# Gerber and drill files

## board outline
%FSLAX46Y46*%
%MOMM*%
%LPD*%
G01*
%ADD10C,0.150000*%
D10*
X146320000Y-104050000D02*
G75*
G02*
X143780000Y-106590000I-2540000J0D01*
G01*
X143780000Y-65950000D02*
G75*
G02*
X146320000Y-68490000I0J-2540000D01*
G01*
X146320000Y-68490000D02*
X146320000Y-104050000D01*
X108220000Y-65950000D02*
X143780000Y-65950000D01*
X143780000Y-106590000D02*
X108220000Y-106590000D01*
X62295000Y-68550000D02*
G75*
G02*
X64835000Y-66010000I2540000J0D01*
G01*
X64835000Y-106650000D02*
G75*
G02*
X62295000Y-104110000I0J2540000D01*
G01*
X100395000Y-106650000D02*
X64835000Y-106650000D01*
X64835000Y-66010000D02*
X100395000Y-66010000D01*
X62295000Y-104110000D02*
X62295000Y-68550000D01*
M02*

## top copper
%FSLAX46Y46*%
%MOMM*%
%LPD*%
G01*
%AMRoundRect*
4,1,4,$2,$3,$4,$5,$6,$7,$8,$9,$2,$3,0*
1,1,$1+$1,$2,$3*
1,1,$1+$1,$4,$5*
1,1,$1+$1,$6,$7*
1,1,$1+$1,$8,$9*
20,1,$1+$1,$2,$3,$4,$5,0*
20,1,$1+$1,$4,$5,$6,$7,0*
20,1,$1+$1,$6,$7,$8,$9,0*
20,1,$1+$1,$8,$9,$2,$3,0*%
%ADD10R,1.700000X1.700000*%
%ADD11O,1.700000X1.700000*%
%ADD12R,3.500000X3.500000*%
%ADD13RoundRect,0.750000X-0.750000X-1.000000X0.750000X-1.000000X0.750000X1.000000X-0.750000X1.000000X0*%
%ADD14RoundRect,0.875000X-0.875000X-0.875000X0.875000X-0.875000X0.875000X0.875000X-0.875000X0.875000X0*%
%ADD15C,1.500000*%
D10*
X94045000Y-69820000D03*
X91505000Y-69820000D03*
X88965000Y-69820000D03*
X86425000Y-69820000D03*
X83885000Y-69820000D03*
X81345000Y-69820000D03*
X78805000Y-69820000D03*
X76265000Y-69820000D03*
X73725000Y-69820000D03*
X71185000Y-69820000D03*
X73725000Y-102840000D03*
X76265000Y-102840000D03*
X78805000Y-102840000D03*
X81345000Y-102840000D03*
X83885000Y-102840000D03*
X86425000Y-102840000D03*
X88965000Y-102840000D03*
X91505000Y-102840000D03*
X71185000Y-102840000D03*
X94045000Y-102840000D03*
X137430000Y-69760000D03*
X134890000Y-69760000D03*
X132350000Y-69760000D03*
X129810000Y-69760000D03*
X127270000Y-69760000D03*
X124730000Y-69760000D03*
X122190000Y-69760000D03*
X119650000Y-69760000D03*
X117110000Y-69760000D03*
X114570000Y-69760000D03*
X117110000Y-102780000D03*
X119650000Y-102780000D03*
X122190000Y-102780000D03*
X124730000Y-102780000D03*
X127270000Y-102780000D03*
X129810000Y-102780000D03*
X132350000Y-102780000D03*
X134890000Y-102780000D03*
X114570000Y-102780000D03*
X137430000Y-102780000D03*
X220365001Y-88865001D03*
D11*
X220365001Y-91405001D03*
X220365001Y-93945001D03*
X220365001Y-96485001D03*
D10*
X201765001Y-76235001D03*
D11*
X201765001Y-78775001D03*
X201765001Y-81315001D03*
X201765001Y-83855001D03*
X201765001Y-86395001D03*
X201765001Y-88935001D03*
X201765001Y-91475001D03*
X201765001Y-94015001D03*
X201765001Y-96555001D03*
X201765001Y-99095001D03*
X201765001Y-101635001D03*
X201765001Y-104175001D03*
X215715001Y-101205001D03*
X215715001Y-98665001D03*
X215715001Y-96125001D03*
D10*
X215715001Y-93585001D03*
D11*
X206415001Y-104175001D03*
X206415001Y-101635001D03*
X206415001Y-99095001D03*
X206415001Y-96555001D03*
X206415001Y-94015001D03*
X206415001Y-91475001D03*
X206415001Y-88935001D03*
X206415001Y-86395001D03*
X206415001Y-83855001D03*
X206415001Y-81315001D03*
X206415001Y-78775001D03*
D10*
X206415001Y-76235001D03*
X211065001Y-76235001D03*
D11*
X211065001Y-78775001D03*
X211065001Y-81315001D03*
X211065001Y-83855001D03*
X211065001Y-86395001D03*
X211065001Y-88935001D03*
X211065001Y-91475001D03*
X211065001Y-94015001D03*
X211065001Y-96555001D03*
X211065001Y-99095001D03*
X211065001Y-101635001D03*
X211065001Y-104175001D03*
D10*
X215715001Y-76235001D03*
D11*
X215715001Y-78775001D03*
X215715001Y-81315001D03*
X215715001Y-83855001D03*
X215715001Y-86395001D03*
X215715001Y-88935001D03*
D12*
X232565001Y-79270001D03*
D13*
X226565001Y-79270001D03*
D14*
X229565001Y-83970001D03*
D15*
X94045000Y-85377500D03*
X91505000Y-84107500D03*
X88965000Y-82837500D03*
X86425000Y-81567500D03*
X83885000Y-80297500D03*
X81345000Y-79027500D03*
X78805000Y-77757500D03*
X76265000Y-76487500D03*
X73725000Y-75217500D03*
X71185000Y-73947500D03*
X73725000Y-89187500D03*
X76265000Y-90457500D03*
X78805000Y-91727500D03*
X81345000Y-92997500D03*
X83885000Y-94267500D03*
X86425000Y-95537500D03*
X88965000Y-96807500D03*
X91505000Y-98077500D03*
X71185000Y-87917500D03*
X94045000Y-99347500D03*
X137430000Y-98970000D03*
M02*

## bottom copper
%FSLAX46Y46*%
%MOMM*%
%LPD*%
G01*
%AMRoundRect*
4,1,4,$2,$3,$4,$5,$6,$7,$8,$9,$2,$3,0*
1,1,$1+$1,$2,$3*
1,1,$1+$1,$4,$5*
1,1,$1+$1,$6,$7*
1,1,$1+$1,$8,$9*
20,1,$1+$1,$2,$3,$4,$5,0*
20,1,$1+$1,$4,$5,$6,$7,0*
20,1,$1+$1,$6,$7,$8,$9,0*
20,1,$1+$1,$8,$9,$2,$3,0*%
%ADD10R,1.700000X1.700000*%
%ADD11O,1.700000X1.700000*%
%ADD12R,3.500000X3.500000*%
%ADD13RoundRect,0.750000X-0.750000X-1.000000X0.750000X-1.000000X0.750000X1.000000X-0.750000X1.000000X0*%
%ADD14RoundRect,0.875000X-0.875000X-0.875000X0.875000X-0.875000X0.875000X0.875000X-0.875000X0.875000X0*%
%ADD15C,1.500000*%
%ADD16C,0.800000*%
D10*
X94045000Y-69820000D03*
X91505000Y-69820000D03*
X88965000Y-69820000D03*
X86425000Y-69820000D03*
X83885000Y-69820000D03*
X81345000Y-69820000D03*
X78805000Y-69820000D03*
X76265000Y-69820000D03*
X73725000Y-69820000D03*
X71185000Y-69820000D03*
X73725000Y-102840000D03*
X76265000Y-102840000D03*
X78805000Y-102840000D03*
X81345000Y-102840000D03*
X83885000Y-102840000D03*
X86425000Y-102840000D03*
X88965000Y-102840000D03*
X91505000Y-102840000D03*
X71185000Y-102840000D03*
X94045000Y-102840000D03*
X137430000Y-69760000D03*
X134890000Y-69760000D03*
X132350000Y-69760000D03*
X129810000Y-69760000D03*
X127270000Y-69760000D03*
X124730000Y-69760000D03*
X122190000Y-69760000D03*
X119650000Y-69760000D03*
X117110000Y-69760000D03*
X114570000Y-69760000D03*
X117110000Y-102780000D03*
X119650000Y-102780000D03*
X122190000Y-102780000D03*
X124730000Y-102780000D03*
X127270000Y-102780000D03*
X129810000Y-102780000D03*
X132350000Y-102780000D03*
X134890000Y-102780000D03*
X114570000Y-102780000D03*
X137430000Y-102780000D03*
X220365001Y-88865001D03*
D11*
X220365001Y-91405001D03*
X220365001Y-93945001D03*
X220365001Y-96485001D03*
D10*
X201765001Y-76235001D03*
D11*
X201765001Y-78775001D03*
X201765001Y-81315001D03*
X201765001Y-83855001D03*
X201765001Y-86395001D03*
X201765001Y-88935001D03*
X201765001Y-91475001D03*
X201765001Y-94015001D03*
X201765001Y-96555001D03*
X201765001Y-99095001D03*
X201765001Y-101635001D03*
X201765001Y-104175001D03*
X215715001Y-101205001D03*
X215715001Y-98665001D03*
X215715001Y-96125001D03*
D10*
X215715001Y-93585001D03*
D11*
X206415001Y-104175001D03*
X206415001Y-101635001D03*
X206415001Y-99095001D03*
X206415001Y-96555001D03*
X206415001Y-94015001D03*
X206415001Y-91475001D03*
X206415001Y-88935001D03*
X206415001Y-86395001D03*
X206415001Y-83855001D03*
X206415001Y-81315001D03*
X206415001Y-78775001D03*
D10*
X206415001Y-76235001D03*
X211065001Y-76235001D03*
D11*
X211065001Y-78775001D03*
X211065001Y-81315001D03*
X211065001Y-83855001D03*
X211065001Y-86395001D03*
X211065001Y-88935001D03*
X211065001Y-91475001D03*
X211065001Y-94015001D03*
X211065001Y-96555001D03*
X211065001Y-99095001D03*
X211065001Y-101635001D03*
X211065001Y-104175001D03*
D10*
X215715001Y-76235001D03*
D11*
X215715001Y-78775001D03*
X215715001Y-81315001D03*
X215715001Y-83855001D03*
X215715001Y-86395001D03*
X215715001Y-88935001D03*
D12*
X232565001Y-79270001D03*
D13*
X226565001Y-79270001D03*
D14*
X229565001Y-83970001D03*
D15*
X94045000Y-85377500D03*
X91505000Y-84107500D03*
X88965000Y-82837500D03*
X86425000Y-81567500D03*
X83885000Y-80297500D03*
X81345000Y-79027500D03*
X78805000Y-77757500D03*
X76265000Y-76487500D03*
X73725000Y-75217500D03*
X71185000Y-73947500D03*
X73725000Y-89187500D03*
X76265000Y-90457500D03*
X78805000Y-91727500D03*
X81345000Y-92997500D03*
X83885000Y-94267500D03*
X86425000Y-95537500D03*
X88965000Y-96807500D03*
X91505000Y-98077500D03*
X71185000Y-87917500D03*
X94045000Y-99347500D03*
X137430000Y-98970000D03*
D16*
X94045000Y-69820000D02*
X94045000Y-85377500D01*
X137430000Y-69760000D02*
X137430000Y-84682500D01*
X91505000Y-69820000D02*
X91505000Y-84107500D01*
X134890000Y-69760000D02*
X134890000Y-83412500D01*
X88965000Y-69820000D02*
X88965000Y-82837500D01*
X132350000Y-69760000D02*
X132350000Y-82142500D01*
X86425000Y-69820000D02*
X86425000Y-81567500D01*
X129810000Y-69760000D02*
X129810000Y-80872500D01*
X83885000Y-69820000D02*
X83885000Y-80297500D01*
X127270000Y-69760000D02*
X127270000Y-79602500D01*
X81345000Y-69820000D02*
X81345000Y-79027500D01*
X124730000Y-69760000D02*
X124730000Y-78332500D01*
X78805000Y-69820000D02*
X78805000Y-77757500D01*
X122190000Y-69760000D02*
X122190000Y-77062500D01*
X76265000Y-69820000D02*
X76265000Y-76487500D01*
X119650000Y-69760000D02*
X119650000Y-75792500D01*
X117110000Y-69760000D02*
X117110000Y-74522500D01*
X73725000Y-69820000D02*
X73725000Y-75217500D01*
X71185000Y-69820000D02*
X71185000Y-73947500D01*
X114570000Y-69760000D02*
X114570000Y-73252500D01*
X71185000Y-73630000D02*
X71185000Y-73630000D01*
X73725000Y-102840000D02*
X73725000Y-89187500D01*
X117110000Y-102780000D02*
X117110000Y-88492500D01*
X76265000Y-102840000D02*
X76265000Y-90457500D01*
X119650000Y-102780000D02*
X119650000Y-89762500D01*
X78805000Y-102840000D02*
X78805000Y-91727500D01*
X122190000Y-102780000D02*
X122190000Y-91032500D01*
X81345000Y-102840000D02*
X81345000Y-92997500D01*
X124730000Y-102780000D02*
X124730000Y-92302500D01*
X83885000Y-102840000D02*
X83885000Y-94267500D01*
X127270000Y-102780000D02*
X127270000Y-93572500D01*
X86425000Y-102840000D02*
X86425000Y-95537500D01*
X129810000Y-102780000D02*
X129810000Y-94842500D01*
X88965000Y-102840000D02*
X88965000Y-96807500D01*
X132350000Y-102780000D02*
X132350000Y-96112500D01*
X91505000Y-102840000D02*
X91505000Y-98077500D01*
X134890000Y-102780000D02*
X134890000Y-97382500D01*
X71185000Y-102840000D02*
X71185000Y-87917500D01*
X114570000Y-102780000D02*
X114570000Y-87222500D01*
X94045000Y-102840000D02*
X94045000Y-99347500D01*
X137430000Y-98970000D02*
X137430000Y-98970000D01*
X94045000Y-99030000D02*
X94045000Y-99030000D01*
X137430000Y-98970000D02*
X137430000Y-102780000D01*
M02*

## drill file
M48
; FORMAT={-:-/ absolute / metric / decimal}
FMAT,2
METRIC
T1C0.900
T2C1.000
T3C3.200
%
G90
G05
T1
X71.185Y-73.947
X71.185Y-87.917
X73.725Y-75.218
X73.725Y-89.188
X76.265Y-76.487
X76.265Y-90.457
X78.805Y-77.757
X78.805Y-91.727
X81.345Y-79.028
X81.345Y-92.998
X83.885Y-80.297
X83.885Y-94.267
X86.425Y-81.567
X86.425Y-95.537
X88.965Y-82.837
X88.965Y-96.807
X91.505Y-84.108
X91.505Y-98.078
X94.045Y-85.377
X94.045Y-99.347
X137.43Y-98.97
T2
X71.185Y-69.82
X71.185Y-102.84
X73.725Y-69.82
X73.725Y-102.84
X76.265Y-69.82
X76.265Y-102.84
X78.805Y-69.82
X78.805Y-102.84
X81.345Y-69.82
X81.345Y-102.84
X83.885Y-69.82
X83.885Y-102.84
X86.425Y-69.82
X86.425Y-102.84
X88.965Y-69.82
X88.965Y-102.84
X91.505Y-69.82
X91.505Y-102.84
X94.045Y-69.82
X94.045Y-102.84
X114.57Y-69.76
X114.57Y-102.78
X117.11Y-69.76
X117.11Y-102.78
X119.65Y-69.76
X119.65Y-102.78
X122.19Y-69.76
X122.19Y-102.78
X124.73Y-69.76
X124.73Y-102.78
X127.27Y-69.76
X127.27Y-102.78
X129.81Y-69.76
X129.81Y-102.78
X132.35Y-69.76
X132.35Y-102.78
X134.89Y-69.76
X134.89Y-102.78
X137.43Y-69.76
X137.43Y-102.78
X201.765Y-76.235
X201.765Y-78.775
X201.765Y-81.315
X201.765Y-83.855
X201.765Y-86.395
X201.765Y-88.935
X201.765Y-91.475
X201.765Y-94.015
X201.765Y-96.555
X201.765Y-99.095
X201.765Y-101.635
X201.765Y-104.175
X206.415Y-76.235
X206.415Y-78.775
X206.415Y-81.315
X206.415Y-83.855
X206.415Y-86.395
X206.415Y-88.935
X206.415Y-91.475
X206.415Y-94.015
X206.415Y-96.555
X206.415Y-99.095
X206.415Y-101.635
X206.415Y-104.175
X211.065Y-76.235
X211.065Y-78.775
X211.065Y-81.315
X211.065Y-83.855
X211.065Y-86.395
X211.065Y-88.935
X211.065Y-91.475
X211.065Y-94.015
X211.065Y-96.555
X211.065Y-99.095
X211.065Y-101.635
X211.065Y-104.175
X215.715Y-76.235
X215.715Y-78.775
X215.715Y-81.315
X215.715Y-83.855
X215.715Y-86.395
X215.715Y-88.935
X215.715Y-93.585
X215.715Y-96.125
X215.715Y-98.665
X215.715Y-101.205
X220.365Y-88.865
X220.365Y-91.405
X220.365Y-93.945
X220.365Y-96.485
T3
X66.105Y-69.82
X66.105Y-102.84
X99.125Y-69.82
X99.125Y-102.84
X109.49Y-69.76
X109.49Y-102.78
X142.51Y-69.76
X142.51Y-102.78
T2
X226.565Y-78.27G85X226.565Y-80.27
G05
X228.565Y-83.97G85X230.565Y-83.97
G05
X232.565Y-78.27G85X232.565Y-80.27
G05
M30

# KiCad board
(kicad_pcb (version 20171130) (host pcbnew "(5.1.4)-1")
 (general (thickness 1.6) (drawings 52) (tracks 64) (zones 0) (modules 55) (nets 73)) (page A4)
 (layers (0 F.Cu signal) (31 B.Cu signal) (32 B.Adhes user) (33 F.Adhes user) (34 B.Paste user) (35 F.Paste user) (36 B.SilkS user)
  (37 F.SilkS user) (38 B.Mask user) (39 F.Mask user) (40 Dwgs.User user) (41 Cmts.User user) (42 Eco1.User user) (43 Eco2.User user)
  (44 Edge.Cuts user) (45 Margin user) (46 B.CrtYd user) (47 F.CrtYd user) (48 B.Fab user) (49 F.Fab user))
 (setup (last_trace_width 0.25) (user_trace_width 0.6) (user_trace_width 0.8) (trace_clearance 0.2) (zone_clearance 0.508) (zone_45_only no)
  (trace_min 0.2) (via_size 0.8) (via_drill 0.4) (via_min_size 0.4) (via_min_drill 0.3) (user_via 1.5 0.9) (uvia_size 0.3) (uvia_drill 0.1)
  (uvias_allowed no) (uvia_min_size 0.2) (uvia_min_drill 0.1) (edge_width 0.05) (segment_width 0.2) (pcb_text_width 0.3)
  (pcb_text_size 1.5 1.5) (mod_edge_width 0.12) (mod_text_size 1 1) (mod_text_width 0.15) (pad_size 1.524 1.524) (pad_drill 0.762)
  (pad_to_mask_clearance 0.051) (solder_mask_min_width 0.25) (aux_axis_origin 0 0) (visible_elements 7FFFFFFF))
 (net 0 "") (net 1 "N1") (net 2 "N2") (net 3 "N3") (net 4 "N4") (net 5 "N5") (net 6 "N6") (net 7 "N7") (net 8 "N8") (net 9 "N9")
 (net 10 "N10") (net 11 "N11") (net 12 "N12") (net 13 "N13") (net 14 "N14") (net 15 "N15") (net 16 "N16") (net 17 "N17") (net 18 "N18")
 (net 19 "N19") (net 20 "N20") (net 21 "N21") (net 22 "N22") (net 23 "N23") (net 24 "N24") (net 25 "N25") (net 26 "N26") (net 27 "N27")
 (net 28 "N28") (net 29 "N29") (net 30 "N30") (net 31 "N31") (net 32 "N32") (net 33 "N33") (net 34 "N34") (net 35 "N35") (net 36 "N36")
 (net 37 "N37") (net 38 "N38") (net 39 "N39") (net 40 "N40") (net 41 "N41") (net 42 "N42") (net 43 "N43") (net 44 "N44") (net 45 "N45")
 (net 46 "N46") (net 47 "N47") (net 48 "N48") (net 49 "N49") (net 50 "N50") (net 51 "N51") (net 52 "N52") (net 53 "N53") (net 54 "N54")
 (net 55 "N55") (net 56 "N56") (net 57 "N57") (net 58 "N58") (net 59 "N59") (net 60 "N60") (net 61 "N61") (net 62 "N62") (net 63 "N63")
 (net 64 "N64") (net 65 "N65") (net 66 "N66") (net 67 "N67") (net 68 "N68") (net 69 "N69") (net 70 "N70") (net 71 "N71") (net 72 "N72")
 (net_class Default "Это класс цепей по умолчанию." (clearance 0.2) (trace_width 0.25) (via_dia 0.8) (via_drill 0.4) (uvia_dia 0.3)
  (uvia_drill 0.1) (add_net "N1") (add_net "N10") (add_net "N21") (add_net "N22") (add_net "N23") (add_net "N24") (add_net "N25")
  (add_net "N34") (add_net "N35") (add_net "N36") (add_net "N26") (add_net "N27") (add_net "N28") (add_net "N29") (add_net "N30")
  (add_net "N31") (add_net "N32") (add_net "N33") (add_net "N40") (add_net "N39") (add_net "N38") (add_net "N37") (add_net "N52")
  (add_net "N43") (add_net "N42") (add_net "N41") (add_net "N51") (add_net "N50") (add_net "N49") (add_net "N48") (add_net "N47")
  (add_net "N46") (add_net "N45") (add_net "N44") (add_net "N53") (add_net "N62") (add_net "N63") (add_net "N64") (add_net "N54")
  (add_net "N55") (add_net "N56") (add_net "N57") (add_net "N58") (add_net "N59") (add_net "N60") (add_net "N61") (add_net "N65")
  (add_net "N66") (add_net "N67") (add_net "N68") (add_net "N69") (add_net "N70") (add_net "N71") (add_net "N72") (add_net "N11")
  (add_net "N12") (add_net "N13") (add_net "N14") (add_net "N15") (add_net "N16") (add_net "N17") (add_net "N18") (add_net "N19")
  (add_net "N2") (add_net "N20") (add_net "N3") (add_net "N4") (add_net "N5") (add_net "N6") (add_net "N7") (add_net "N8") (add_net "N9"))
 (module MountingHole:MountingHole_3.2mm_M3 (layer F.Cu) (at 142.51 102.78 90)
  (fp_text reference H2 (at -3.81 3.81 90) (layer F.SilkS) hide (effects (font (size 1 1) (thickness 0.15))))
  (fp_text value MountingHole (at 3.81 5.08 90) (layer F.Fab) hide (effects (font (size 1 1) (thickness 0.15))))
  (pad 1 np_thru_hole circle (at 0 0 90) (size 3.2 3.2) (drill 3.2) (layers *.Cu *.Mask)))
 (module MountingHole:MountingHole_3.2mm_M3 (layer F.Cu) (at 142.51 69.76 90)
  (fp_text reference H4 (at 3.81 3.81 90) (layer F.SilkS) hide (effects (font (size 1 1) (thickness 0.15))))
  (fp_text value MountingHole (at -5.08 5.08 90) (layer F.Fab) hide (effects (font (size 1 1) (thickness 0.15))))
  (pad 1 np_thru_hole circle (at 0 0 90) (size 3.2 3.2) (drill 3.2) (layers *.Cu *.Mask)))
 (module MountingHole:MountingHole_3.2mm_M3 (layer F.Cu) (at 109.49 102.78 90)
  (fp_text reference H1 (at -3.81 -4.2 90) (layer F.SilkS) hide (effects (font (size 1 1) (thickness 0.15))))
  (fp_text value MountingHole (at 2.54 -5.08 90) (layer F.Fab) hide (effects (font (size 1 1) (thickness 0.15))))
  (pad 1 np_thru_hole circle (at 0 0 90) (size 3.2 3.2) (drill 3.2) (layers *.Cu *.Mask)))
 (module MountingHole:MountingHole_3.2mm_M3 (layer F.Cu) (at 109.49 69.76 90)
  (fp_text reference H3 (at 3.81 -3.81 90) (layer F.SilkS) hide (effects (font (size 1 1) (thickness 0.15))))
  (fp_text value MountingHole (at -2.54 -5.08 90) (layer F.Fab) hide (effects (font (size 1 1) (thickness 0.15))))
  (pad 1 np_thru_hole circle (at 0 0 90) (size 3.2 3.2) (drill 3.2) (layers *.Cu *.Mask)))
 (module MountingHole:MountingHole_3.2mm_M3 (layer F.Cu) (at 66.105 102.84 90)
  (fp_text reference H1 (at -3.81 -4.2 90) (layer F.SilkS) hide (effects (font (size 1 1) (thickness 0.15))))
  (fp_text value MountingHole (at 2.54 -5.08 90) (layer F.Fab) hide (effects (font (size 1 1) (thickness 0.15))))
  (pad 1 np_thru_hole circle (at 0 0 90) (size 3.2 3.2) (drill 3.2) (layers *.Cu *.Mask)))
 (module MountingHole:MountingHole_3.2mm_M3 (layer F.Cu) (at 99.125 102.84 90)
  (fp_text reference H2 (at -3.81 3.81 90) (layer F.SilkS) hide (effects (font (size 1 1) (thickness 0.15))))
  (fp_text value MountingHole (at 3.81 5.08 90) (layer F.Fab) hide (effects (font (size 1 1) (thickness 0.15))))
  (pad 1 np_thru_hole circle (at 0 0 90) (size 3.2 3.2) (drill 3.2) (layers *.Cu *.Mask)))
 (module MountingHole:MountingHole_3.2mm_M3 (layer F.Cu) (at 66.105 69.82 90)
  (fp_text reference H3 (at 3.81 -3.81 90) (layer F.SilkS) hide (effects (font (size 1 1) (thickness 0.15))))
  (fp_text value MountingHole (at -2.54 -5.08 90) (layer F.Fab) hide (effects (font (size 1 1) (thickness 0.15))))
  (pad 1 np_thru_hole circle (at 0 0 90) (size 3.2 3.2) (drill 3.2) (layers *.Cu *.Mask)))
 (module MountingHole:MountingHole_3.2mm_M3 (layer F.Cu) (at 99.125 69.82 90)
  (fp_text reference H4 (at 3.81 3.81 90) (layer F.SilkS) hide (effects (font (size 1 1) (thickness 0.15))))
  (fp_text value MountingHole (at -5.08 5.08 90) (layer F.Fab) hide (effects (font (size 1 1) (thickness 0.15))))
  (pad 1 np_thru_hole circle (at 0 0 90) (size 3.2 3.2) (drill 3.2) (layers *.Cu *.Mask)))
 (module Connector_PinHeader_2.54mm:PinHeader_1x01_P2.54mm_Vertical (layer F.Cu) (at 94.045 69.82 90)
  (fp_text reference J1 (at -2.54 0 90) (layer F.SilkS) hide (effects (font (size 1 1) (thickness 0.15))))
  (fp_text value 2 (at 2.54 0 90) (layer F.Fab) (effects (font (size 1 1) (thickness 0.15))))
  (pad 1 thru_hole rect (at 0 0 90) (size 1.7 1.7) (drill 1) (layers *.Cu *.Mask) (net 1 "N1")))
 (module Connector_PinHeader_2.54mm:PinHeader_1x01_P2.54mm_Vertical (layer F.Cu) (at 91.505 69.82 90)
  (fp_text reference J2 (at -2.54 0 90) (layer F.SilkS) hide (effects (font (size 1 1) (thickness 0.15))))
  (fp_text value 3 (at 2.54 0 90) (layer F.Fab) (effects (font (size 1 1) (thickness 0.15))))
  (pad 1 thru_hole rect (at 0 0 90) (size 1.7 1.7) (drill 1) (layers *.Cu *.Mask) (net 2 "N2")))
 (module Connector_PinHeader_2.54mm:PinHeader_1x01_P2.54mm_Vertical (layer F.Cu) (at 88.965 69.82 90)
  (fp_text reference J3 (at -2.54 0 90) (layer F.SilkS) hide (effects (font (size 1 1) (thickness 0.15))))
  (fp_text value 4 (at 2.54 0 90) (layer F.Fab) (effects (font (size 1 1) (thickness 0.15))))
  (pad 1 thru_hole rect (at 0 0 90) (size 1.7 1.7) (drill 1) (layers *.Cu *.Mask) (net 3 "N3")))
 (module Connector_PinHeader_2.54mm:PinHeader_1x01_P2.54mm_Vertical (layer F.Cu) (at 86.425 69.82 90)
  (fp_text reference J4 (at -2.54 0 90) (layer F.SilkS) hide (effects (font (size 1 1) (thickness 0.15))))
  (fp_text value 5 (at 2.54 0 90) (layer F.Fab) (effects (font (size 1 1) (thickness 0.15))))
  (pad 1 thru_hole rect (at 0 0 90) (size 1.7 1.7) (drill 1) (layers *.Cu *.Mask) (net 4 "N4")))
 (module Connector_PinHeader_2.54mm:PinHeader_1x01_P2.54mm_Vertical (layer F.Cu) (at 83.885 69.82 90)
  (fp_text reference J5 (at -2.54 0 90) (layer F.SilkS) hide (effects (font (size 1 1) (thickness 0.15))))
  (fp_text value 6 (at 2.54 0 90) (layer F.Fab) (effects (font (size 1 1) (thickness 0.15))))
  (pad 1 thru_hole rect (at 0 0 90) (size 1.7 1.7) (drill 1) (layers *.Cu *.Mask) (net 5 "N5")))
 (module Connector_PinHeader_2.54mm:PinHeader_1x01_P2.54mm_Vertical (layer F.Cu) (at 81.345 69.82 90)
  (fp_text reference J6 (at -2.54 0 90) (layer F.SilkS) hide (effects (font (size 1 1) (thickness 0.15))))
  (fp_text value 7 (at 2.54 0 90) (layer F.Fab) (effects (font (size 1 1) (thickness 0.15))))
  (pad 1 thru_hole rect (at 0 0 90) (size 1.7 1.7) (drill 1) (layers *.Cu *.Mask) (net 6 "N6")))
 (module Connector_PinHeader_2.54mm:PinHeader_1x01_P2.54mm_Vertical (layer F.Cu) (at 78.805 69.82 90)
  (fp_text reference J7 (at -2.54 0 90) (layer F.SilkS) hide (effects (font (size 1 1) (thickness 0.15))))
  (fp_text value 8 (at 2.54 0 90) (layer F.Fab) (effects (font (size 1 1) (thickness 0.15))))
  (pad 1 thru_hole rect (at 0 0 90) (size 1.7 1.7) (drill 1) (layers *.Cu *.Mask) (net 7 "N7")))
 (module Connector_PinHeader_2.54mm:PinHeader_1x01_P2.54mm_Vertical (layer F.Cu) (at 76.265 69.82 90)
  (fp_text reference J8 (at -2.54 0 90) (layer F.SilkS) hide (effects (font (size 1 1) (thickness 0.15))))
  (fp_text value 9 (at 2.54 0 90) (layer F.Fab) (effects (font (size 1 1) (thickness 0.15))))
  (pad 1 thru_hole rect (at 0 0 90) (size 1.7 1.7) (drill 1) (layers *.Cu *.Mask) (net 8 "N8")))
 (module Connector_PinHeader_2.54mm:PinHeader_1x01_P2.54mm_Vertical (layer F.Cu) (at 73.725 69.82 90)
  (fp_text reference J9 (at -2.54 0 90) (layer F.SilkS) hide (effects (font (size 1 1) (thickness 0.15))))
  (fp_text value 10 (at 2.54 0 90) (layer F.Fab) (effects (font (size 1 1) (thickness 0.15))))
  (pad 1 thru_hole rect (at 0 0 90) (size 1.7 1.7) (drill 1) (layers *.Cu *.Mask) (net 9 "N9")))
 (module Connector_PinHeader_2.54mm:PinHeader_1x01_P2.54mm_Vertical (layer F.Cu) (at 71.185 69.82 90)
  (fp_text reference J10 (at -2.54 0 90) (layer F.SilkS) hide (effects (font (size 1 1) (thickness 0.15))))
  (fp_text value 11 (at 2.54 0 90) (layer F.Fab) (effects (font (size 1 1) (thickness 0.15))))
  (pad 1 thru_hole rect (at 0 0 90) (size 1.7 1.7) (drill 1) (layers *.Cu *.Mask) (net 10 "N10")))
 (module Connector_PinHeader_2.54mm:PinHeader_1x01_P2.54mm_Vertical (layer F.Cu) (at 73.725 102.84 90)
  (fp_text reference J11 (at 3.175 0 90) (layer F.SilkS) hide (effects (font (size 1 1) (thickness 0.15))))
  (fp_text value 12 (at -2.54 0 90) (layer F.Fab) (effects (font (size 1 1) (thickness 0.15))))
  (pad 1 thru_hole rect (at 0 0 90) (size 1.7 1.7) (drill 1) (layers *.Cu *.Mask) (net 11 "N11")))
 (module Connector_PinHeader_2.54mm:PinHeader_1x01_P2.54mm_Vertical (layer F.Cu) (at 76.265 102.84 90)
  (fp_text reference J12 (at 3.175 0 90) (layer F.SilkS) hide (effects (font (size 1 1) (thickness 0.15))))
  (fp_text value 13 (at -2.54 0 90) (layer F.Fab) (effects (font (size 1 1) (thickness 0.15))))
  (pad 1 thru_hole rect (at 0 0 90) (size 1.7 1.7) (drill 1) (layers *.Cu *.Mask) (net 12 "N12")))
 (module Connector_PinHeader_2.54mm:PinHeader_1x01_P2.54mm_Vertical (layer F.Cu) (at 78.805 102.84 90)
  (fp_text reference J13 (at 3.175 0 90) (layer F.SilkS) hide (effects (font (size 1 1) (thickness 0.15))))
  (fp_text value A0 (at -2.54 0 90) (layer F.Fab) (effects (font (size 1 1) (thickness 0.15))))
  (pad 1 thru_hole rect (at 0 0 90) (size 1.7 1.7) (drill 1) (layers *.Cu *.Mask) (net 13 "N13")))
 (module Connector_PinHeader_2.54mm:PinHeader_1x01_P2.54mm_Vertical (layer F.Cu) (at 81.345 102.84 90)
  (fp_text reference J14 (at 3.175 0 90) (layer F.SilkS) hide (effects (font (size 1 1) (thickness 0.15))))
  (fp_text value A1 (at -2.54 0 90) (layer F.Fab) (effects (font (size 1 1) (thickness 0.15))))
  (pad 1 thru_hole rect (at 0 0 90) (size 1.7 1.7) (drill 1) (layers *.Cu *.Mask) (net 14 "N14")))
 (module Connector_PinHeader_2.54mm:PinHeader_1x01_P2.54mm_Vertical (layer F.Cu) (at 83.885 102.84 90)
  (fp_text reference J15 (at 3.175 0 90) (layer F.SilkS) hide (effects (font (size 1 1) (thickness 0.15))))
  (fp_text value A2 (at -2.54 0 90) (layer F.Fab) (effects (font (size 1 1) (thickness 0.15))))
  (pad 1 thru_hole rect (at 0 0 90) (size 1.7 1.7) (drill 1) (layers *.Cu *.Mask) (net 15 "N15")))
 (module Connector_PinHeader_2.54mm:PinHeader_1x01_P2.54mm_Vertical (layer F.Cu) (at 86.425 102.84 90)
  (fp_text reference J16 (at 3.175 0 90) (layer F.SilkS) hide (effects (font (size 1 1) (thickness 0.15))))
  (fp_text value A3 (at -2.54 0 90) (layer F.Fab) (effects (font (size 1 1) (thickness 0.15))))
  (pad 1 thru_hole rect (at 0 0 90) (size 1.7 1.7) (drill 1) (layers *.Cu *.Mask) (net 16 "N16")))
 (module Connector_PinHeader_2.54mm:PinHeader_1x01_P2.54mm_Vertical (layer F.Cu) (at 88.965 102.84 90)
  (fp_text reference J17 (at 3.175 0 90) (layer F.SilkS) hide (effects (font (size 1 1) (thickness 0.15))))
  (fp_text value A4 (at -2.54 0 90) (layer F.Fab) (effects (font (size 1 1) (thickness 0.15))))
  (pad 1 thru_hole rect (at 0 0 90) (size 1.7 1.7) (drill 1) (layers *.Cu *.Mask) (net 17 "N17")))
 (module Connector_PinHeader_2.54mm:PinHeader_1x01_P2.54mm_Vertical (layer F.Cu) (at 91.505 102.84 90)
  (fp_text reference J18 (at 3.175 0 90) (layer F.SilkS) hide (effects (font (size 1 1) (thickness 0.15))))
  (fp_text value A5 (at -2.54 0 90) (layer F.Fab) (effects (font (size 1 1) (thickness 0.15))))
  (pad 1 thru_hole rect (at 0 0 90) (size 1.7 1.7) (drill 1) (layers *.Cu *.Mask) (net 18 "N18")))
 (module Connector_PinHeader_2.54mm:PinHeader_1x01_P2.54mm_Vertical (layer F.Cu) (at 71.185 102.84 90)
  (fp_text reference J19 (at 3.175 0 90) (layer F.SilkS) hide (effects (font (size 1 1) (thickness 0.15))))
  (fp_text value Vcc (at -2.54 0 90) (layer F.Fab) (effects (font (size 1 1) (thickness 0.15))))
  (pad 1 thru_hole rect (at 0 0 90) (size 1.7 1.7) (drill 1) (layers *.Cu *.Mask) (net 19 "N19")))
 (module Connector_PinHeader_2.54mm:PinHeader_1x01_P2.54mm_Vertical (layer F.Cu) (at 94.045 102.84 90)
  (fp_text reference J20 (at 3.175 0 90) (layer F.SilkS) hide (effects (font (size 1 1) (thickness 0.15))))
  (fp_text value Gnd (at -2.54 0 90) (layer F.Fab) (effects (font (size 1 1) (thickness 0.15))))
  (pad 1 thru_hole rect (at 0 0 90) (size 1.7 1.7) (drill 1) (layers *.Cu *.Mask) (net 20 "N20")))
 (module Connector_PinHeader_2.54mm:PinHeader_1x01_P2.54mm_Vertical (layer F.Cu) (at 137.43 69.76 90)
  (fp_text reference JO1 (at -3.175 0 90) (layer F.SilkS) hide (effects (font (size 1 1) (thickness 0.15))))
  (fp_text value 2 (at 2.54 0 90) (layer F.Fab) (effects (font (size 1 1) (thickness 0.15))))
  (pad 1 thru_hole rect (at 0 0 90) (size 1.7 1.7) (drill 1) (layers *.Cu *.Mask) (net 1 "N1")))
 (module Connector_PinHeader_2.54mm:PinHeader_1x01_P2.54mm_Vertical (layer F.Cu) (at 134.89 69.76 90)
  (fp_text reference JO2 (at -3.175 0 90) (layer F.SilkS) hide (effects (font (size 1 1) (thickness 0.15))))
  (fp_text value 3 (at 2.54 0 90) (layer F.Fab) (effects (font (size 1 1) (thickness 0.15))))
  (pad 1 thru_hole rect (at 0 0 90) (size 1.7 1.7) (drill 1) (layers *.Cu *.Mask) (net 2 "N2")))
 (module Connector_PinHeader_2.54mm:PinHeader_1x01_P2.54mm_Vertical (layer F.Cu) (at 132.35 69.76 90)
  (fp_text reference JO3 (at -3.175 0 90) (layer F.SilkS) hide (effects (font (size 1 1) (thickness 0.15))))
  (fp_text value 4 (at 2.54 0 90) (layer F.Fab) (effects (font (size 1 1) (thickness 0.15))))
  (pad 1 thru_hole rect (at 0 0 90) (size 1.7 1.7) (drill 1) (layers *.Cu *.Mask) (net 3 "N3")))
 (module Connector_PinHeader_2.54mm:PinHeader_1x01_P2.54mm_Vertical (layer F.Cu) (at 129.81 69.76 90)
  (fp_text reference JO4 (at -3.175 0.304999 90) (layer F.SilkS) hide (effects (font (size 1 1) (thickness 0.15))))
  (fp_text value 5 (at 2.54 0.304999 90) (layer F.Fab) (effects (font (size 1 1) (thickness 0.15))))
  (pad 1 thru_hole rect (at 0 0 90) (size 1.7 1.7) (drill 1) (layers *.Cu *.Mask) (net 4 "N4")))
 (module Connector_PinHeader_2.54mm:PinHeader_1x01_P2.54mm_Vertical (layer F.Cu) (at 127.27 69.76 90)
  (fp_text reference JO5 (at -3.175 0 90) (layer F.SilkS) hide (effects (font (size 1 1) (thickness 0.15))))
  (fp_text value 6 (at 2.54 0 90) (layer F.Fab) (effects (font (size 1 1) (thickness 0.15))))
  (pad 1 thru_hole rect (at 0 0 90) (size 1.7 1.7) (drill 1) (layers *.Cu *.Mask) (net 5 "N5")))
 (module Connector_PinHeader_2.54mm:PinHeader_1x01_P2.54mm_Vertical (layer F.Cu) (at 124.73 69.76 90)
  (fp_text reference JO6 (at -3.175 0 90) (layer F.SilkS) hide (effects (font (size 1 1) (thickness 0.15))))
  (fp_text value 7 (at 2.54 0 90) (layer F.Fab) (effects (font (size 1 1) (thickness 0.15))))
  (pad 1 thru_hole rect (at 0 0 90) (size 1.7 1.7) (drill 1) (layers *.Cu *.Mask) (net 6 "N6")))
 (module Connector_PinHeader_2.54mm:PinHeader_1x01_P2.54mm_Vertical (layer F.Cu) (at 122.19 69.76 90)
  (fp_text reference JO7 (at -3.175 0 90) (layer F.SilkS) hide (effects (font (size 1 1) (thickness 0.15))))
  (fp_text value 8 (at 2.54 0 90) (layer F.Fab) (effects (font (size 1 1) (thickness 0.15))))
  (pad 1 thru_hole rect (at 0 0 90) (size 1.7 1.7) (drill 1) (layers *.Cu *.Mask) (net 7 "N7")))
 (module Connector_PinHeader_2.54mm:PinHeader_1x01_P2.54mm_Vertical (layer F.Cu) (at 119.65 69.76 90)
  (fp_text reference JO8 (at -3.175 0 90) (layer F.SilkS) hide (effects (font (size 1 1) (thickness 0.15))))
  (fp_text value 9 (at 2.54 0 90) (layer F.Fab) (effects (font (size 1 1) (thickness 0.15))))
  (pad 1 thru_hole rect (at 0 0 90) (size 1.7 1.7) (drill 1) (layers *.Cu *.Mask) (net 8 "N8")))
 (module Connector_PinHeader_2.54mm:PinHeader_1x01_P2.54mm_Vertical (layer F.Cu) (at 117.11 69.76 90)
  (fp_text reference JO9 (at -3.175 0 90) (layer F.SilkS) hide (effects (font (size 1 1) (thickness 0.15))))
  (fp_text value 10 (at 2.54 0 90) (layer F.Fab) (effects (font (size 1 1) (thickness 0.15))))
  (pad 1 thru_hole rect (at 0 0 90) (size 1.7 1.7) (drill 1) (layers *.Cu *.Mask) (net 9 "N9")))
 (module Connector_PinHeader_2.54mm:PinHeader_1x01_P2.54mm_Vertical (layer F.Cu) (at 114.57 69.76 90)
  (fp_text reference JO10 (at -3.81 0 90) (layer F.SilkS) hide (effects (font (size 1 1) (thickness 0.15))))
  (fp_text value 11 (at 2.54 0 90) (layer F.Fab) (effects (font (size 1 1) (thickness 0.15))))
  (pad 1 thru_hole rect (at 0 0 90) (size 1.7 1.7) (drill 1) (layers *.Cu *.Mask) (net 10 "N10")))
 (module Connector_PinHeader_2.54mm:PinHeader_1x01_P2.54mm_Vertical (layer F.Cu) (at 117.11 102.78 90)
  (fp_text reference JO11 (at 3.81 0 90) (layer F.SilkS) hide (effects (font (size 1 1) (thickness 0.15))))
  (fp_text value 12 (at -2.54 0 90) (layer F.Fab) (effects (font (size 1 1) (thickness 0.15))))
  (pad 1 thru_hole rect (at 0 0 90) (size 1.7 1.7) (drill 1) (layers *.Cu *.Mask) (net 11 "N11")))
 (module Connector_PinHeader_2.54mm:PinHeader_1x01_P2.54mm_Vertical (layer F.Cu) (at 119.65 102.78 90)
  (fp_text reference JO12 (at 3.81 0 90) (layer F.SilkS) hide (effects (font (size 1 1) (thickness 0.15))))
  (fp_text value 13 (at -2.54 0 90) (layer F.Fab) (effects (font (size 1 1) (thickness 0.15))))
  (pad 1 thru_hole rect (at 0 0 90) (size 1.7 1.7) (drill 1) (layers *.Cu *.Mask) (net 12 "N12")))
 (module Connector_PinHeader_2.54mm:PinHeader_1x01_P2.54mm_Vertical (layer F.Cu) (at 122.19 102.78 90)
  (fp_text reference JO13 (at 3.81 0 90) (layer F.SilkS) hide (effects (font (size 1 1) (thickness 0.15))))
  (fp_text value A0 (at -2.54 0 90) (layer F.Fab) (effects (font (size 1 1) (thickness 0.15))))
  (pad 1 thru_hole rect (at 0 0 90) (size 1.7 1.7) (drill 1) (layers *.Cu *.Mask) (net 13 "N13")))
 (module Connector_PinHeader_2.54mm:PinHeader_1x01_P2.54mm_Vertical (layer F.Cu) (at 124.73 102.78 90)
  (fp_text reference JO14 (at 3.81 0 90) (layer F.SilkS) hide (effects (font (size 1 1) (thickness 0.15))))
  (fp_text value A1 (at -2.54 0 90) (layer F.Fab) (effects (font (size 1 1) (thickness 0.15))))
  (pad 1 thru_hole rect (at 0 0 90) (size 1.7 1.7) (drill 1) (layers *.Cu *.Mask) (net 14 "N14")))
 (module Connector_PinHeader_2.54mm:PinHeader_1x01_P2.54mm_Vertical (layer F.Cu) (at 127.27 102.78 90)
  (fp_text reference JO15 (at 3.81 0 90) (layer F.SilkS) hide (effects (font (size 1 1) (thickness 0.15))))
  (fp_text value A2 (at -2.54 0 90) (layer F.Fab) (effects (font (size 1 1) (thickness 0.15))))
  (pad 1 thru_hole rect (at 0 0 90) (size 1.7 1.7) (drill 1) (layers *.Cu *.Mask) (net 15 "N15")))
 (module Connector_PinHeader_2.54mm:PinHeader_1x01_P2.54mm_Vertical (layer F.Cu) (at 129.81 102.78 90)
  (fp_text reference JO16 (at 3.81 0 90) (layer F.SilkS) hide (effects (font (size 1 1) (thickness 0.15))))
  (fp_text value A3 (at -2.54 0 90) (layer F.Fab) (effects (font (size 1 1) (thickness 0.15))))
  (pad 1 thru_hole rect (at 0 0 90) (size 1.7 1.7) (drill 1) (layers *.Cu *.Mask) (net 16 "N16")))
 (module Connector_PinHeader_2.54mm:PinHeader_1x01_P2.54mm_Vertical (layer F.Cu) (at 132.35 102.78 90)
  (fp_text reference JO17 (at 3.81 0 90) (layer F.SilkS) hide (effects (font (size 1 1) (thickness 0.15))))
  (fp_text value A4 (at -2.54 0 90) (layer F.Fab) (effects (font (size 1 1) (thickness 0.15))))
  (pad 1 thru_hole rect (at 0 0 90) (size 1.7 1.7) (drill 1) (layers *.Cu *.Mask) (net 17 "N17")))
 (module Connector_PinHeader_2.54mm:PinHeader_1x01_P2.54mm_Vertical (layer F.Cu) (at 134.89 102.78 90)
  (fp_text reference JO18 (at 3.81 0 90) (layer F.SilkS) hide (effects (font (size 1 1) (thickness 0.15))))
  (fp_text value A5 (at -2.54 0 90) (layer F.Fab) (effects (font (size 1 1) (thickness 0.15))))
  (pad 1 thru_hole rect (at 0 0 90) (size 1.7 1.7) (drill 1) (layers *.Cu *.Mask) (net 18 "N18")))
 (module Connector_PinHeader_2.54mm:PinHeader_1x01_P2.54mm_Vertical (layer F.Cu) (at 114.57 102.78 90)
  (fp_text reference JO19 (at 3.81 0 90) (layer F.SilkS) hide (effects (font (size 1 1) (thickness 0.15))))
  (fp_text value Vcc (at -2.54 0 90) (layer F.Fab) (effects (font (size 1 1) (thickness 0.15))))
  (pad 1 thru_hole rect (at 0 0 90) (size 1.7 1.7) (drill 1) (layers *.Cu *.Mask) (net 19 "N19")))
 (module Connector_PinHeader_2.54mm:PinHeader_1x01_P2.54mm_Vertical (layer F.Cu) (at 137.43 102.78 90)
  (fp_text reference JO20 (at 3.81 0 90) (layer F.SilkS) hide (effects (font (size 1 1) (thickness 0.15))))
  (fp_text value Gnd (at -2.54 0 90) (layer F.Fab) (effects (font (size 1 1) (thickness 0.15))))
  (pad 1 thru_hole rect (at 0 0 90) (size 1.7 1.7) (drill 1) (layers *.Cu *.Mask) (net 20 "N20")))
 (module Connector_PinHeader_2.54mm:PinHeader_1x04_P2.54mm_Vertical (layer F.Cu) (at 220.365001 88.865001)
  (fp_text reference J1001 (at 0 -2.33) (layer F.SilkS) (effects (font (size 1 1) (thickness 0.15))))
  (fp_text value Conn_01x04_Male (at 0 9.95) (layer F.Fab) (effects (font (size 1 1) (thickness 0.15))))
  (pad 1 thru_hole rect (at 0 0) (size 1.7 1.7) (drill 1) (layers *.Cu *.Mask) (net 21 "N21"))
  (pad 2 thru_hole oval (at 0 2.54) (size 1.7 1.7) (drill 1) (layers *.Cu *.Mask) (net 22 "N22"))
  (pad 3 thru_hole oval (at 0 5.08) (size 1.7 1.7) (drill 1) (layers *.Cu *.Mask) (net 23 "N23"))
  (pad 4 thru_hole oval (at 0 7.62) (size 1.7 1.7) (drill 1) (layers *.Cu *.Mask) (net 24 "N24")))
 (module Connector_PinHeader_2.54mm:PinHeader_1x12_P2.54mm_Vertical (layer F.Cu) (at 201.765001 76.235001)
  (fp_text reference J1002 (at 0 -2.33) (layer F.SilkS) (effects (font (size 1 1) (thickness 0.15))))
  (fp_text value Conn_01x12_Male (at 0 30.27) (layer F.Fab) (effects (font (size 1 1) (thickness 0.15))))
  (pad 1 thru_hole rect (at 0 0) (size 1.7 1.7) (drill 1) (layers *.Cu *.Mask) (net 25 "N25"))
  (pad 2 thru_hole oval (at 0 2.54) (size 1.7 1.7) (drill 1) (layers *.Cu *.Mask) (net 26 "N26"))
  (pad 3 thru_hole oval (at 0 5.08) (size 1.7 1.7) (drill 1) (layers *.Cu *.Mask) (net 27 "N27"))
  (pad 4 thru_hole oval (at 0 7.62) (size 1.7 1.7) (drill 1) (layers *.Cu *.Mask) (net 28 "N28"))
  (pad 5 thru_hole oval (at 0 10.16) (size 1.7 1.7) (drill 1) (layers *.Cu *.Mask) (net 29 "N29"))
  (pad 6 thru_hole oval (at 0 12.7) (size 1.7 1.7) (drill 1) (layers *.Cu *.Mask) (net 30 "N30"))
  (pad 7 thru_hole oval (at 0 15.24) (size 1.7 1.7) (drill 1) (layers *.Cu *.Mask) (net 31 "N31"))
  (pad 8 thru_hole oval (at 0 17.78) (size 1.7 1.7) (drill 1) (layers *.Cu *.Mask) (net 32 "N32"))
  (pad 9 thru_hole oval (at 0 20.32) (size 1.7 1.7) (drill 1) (layers *.Cu *.Mask) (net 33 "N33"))
  (pad 10 thru_hole oval (at 0 22.86) (size 1.7 1.7) (drill 1) (layers *.Cu *.Mask) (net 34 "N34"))
  (pad 11 thru_hole oval (at 0 25.4) (size 1.7 1.7) (drill 1) (layers *.Cu *.Mask) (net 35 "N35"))
  (pad 12 thru_hole oval (at 0 27.94) (size 1.7 1.7) (drill 1) (layers *.Cu *.Mask) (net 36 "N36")))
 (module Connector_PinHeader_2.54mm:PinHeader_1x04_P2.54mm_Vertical (layer F.Cu) (at 215.715001 93.585001)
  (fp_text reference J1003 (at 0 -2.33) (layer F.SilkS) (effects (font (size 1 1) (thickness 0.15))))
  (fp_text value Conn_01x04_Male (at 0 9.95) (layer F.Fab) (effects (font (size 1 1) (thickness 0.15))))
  (pad 4 thru_hole oval (at 0 7.62) (size 1.7 1.7) (drill 1) (layers *.Cu *.Mask) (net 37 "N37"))
  (pad 3 thru_hole oval (at 0 5.08) (size 1.7 1.7) (drill 1) (layers *.Cu *.Mask) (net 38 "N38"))
  (pad 2 thru_hole oval (at 0 2.54) (size 1.7 1.7) (drill 1) (layers *.Cu *.Mask) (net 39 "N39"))
  (pad 1 thru_hole rect (at 0 0) (size 1.7 1.7) (drill 1) (layers *.Cu *.Mask) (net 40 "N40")))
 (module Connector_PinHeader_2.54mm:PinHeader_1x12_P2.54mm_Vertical (layer F.Cu) (at 206.415001 76.235001)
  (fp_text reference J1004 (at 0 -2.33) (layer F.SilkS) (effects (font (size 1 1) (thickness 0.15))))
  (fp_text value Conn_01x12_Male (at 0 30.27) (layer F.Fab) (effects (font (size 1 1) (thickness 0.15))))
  (pad 12 thru_hole oval (at 0 27.94) (size 1.7 1.7) (drill 1) (layers *.Cu *.Mask) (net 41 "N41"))
  (pad 11 thru_hole oval (at 0 25.4) (size 1.7 1.7) (drill 1) (layers *.Cu *.Mask) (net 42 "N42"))
  (pad 10 thru_hole oval (at 0 22.86) (size 1.7 1.7) (drill 1) (layers *.Cu *.Mask) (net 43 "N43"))
  (pad 9 thru_hole oval (at 0 20.32) (size 1.7 1.7) (drill 1) (layers *.Cu *.Mask) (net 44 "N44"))
  (pad 8 thru_hole oval (at 0 17.78) (size 1.7 1.7) (drill 1) (layers *.Cu *.Mask) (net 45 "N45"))
  (pad 7 thru_hole oval (at 0 15.24) (size 1.7 1.7) (drill 1) (layers *.Cu *.Mask) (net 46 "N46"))
  (pad 6 thru_hole oval (at 0 12.7) (size 1.7 1.7) (drill 1) (layers *.Cu *.Mask) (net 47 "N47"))
  (pad 5 thru_hole oval (at 0 10.16) (size 1.7 1.7) (drill 1) (layers *.Cu *.Mask) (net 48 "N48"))
  (pad 4 thru_hole oval (at 0 7.62) (size 1.7 1.7) (drill 1) (layers *.Cu *.Mask) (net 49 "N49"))
  (pad 3 thru_hole oval (at 0 5.08) (size 1.7 1.7) (drill 1) (layers *.Cu *.Mask) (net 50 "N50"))
  (pad 2 thru_hole oval (at 0 2.54) (size 1.7 1.7) (drill 1) (layers *.Cu *.Mask) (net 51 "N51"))
  (pad 1 thru_hole rect (at 0 0) (size 1.7 1.7) (drill 1) (layers *.Cu *.Mask) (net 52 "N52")))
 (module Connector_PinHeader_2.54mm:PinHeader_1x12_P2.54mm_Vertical (layer F.Cu) (at 211.065001 76.235001)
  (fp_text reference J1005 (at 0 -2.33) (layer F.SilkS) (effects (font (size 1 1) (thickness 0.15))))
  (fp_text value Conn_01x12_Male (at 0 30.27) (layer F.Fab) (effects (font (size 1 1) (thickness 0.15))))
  (pad 1 thru_hole rect (at 0 0) (size 1.7 1.7) (drill 1) (layers *.Cu *.Mask) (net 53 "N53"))
  (pad 2 thru_hole oval (at 0 2.54) (size 1.7 1.7) (drill 1) (layers *.Cu *.Mask) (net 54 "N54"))
  (pad 3 thru_hole oval (at 0 5.08) (size 1.7 1.7) (drill 1) (layers *.Cu *.Mask) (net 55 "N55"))
  (pad 4 thru_hole oval (at 0 7.62) (size 1.7 1.7) (drill 1) (layers *.Cu *.Mask) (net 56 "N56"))
  (pad 5 thru_hole oval (at 0 10.16) (size 1.7 1.7) (drill 1) (layers *.Cu *.Mask) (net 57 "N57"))
  (pad 6 thru_hole oval (at 0 12.7) (size 1.7 1.7) (drill 1) (layers *.Cu *.Mask) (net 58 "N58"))
  (pad 7 thru_hole oval (at 0 15.24) (size 1.7 1.7) (drill 1) (layers *.Cu *.Mask) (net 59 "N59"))
  (pad 8 thru_hole oval (at 0 17.78) (size 1.7 1.7) (drill 1) (layers *.Cu *.Mask) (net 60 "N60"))
  (pad 9 thru_hole oval (at 0 20.32) (size 1.7 1.7) (drill 1) (layers *.Cu *.Mask) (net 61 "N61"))
  (pad 10 thru_hole oval (at 0 22.86) (size 1.7 1.7) (drill 1) (layers *.Cu *.Mask) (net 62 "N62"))
  (pad 11 thru_hole oval (at 0 25.4) (size 1.7 1.7) (drill 1) (layers *.Cu *.Mask) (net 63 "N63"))
  (pad 12 thru_hole oval (at 0 27.94) (size 1.7 1.7) (drill 1) (layers *.Cu *.Mask) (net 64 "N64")))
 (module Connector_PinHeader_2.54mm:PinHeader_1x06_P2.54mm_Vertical (layer F.Cu) (at 215.715001 76.235001)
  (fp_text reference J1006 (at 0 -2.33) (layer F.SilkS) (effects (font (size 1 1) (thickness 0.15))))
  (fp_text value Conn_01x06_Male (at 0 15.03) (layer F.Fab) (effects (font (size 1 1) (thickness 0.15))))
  (pad 1 thru_hole rect (at 0 0) (size 1.7 1.7) (drill 1) (layers *.Cu *.Mask) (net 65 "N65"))
  (pad 2 thru_hole oval (at 0 2.54) (size 1.7 1.7) (drill 1) (layers *.Cu *.Mask) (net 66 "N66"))
  (pad 3 thru_hole oval (at 0 5.08) (size 1.7 1.7) (drill 1) (layers *.Cu *.Mask) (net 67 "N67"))
  (pad 4 thru_hole oval (at 0 7.62) (size 1.7 1.7) (drill 1) (layers *.Cu *.Mask) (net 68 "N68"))
  (pad 5 thru_hole oval (at 0 10.16) (size 1.7 1.7) (drill 1) (layers *.Cu *.Mask) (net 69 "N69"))
  (pad 6 thru_hole oval (at 0 12.7) (size 1.7 1.7) (drill 1) (layers *.Cu *.Mask) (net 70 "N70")))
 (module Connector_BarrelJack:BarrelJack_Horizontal (layer F.Cu) (at 232.565001 79.270001)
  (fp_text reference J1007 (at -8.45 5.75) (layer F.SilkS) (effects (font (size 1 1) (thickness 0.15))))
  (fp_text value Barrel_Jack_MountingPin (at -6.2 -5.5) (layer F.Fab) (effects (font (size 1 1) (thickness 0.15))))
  (pad 1 thru_hole rect (at 0 0) (size 3.5 3.5) (drill oval 1 3) (layers *.Cu *.Mask) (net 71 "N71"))
  (pad 2 thru_hole roundrect (at -6 0) (size 3 3.5) (drill oval 1 3) (layers *.Cu *.Mask) (roundrect_rratio 0.25) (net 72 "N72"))
  (pad 3 thru_hole roundrect (at -3 4.7) (size 3.5 3.5) (drill oval 3 1) (layers *.Cu *.Mask) (roundrect_rratio 0.25)))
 (gr_arc (start 143.78 104.05) (end 143.78 106.59) (angle -90) (layer Edge.Cuts) (width 0.15))
 (gr_arc (start 143.78 68.49) (end 146.32 68.49) (angle -90) (layer Edge.Cuts) (width 0.15))
 (gr_line (start 146.32 68.49) (end 146.32 104.05) (layer Edge.Cuts) (width 0.15))
 (gr_line (start 108.22 65.95) (end 143.78 65.95) (layer Edge.Cuts) (width 0.15))
 (gr_line (start 143.78 106.59) (end 108.22 106.59) (layer Edge.Cuts) (width 0.15))
 (gr_arc (start 64.835 68.55) (end 64.835 66.01) (angle -90) (layer Edge.Cuts) (width 0.15))
 (gr_arc (start 64.835 104.11) (end 62.295 104.11) (angle -90) (layer Edge.Cuts) (width 0.15))
 (gr_line (start 100.395 106.65) (end 64.835 106.65) (layer Edge.Cuts) (width 0.15))
 (gr_line (start 64.835 66.01) (end 100.395 66.01) (layer Edge.Cuts) (width 0.15))
 (gr_line (start 62.295 104.11) (end 62.295 68.55) (layer Edge.Cuts) (width 0.15))
 (segment (start 94.045 69.82) (end 94.045 85.3775) (width 0.8) (layer B.Cu) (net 1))
 (via (at 94.045 85.3775) (size 1.5) (drill 0.9) (layers F.Cu B.Cu) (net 1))
 (segment (start 137.43 69.76) (end 137.43 84.6825) (width 0.8) (layer B.Cu) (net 1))
 (segment (start 91.505 69.82) (end 91.505 84.1075) (width 0.8) (layer B.Cu) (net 2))
 (via (at 91.505 84.1075) (size 1.5) (drill 0.9) (layers F.Cu B.Cu) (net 2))
 (segment (start 134.89 69.76) (end 134.89 83.4125) (width 0.8) (layer B.Cu) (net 2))
 (segment (start 88.965 69.82) (end 88.965 82.8375) (width 0.8) (layer B.Cu) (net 3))
 (via (at 88.965 82.8375) (size 1.5) (drill 0.9) (layers F.Cu B.Cu) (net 3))
 (segment (start 132.35 69.76) (end 132.35 82.1425) (width 0.8) (layer B.Cu) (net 3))
 (segment (start 86.425 69.82) (end 86.425 81.5675) (width 0.8) (layer B.Cu) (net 4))
 (via (at 86.425 81.5675) (size 1.5) (drill 0.9) (layers F.Cu B.Cu) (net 4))
 (segment (start 129.81 69.76) (end 129.81 80.8725) (width 0.8) (layer B.Cu) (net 4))
 (segment (start 83.885 69.82) (end 83.885 80.2975) (width 0.8) (layer B.Cu) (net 5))
 (via (at 83.885 80.2975) (size 1.5) (drill 0.9) (layers F.Cu B.Cu) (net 5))
 (segment (start 127.27 69.76) (end 127.27 79.6025) (width 0.8) (layer B.Cu) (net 5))
 (segment (start 81.345 69.82) (end 81.345 79.0275) (width 0.8) (layer B.Cu) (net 6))
 (via (at 81.345 79.0275) (size 1.5) (drill 0.9) (layers F.Cu B.Cu) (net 6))
 (segment (start 124.73 69.76) (end 124.73 78.3325) (width 0.8) (layer B.Cu) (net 6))
 (segment (start 78.805 69.82) (end 78.805 77.7575) (width 0.8) (layer B.Cu) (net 7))
 (via (at 78.805 77.7575) (size 1.5) (drill 0.9) (layers F.Cu B.Cu) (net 7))
 (segment (start 122.19 69.76) (end 122.19 77.0625) (width 0.8) (layer B.Cu) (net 7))
 (segment (start 76.265 69.82) (end 76.265 76.4875) (width 0.8) (layer B.Cu) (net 8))
 (segment (start 119.65 69.76) (end 119.65 75.7925) (width 0.8) (layer B.Cu) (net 8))
 (via (at 76.265 76.4875) (size 1.5) (drill 0.9) (layers F.Cu B.Cu) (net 8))
 (segment (start 117.11 69.76) (end 117.11 74.5225) (width 0.8) (layer B.Cu) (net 9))
 (segment (start 73.725 69.82) (end 73.725 75.2175) (width 0.8) (layer B.Cu) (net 9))
 (via (at 73.725 75.2175) (size 1.5) (drill 0.9) (layers F.Cu B.Cu) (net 9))
 (segment (start 71.185 69.82) (end 71.185 73.9475) (width 0.8) (layer B.Cu) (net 10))
 (segment (start 114.57 69.76) (end 114.57 73.2525) (width 0.8) (layer B.Cu) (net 10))
 (segment (start 71.185 73.63) (end 71.185 73.63) (width 0.8) (layer B.Cu) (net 10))
 (via (at 71.185 73.9475) (size 1.5) (drill 0.9) (layers F.Cu B.Cu) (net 10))
 (via (at 73.725 89.1875) (size 1.5) (drill 0.9) (layers F.Cu B.Cu) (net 11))
 (segment (start 73.725 102.84) (end 73.725 89.1875) (width 0.8) (layer B.Cu) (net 11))
 (segment (start 117.11 102.78) (end 117.11 88.4925) (width 0.8) (layer B.Cu) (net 11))
 (via (at 76.265 90.4575) (size 1.5) (drill 0.9) (layers F.Cu B.Cu) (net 12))
 (segment (start 76.265 102.84) (end 76.265 90.4575) (width 0.8) (layer B.Cu) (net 12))
 (segment (start 119.65 102.78) (end 119.65 89.7625) (width 0.8) (layer B.Cu) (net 12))
 (via (at 78.805 91.7275) (size 1.5) (drill 0.9) (layers F.Cu B.Cu) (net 13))
 (segment (start 78.805 102.84) (end 78.805 91.7275) (width 0.8) (layer B.Cu) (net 13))
 (segment (start 122.19 102.78) (end 122.19 91.0325) (width 0.8) (layer B.Cu) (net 13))
 (via (at 81.345 92.9975) (size 1.5) (drill 0.9) (layers F.Cu B.Cu) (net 14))
 (segment (start 81.345 102.84) (end 81.345 92.9975) (width 0.8) (layer B.Cu) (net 14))
 (segment (start 124.73 102.78) (end 124.73 92.3025) (width 0.8) (layer B.Cu) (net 14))
 (via (at 83.885 94.2675) (size 1.5) (drill 0.9) (layers F.Cu B.Cu) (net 15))
 (segment (start 83.885 102.84) (end 83.885 94.2675) (width 0.8) (layer B.Cu) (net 15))
 (segment (start 127.27 102.78) (end 127.27 93.5725) (width 0.8) (layer B.Cu) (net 15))
 (via (at 86.425 95.5375) (size 1.5) (drill 0.9) (layers F.Cu B.Cu) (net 16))
 (segment (start 86.425 102.84) (end 86.425 95.5375) (width 0.8) (layer B.Cu) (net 16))
 (segment (start 129.81 102.78) (end 129.81 94.8425) (width 0.8) (layer B.Cu) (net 16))
 (via (at 88.965 96.8075) (size 1.5) (drill 0.9) (layers F.Cu B.Cu) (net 17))
 (segment (start 88.965 102.84) (end 88.965 96.8075) (width 0.8) (layer B.Cu) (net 17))
 (segment (start 132.35 102.78) (end 132.35 96.1125) (width 0.8) (layer B.Cu) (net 17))
 (via (at 91.505 98.0775) (size 1.5) (drill 0.9) (layers F.Cu B.Cu) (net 18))
 (segment (start 91.505 102.84) (end 91.505 98.0775) (width 0.8) (layer B.Cu) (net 18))
 (segment (start 134.89 102.78) (end 134.89 97.3825) (width 0.8) (layer B.Cu) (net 18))
 (via (at 71.185 87.9175) (size 1.5) (drill 0.9) (layers F.Cu B.Cu) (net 19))
 (segment (start 71.185 102.84) (end 71.185 87.9175) (width 0.8) (layer B.Cu) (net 19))
 (segment (start 114.57 102.78) (end 114.57 87.2225) (width 0.8) (layer B.Cu) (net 19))
 (segment (start 94.045 102.84) (end 94.045 99.3475) (width 0.8) (layer B.Cu) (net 20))
 (segment (start 137.43 98.97) (end 137.43 98.97) (width 0.8) (layer B.Cu) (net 20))
 (segment (start 94.045 99.03) (end 94.045 99.03) (width 0.8) (layer B.Cu) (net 20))
 (via (at 94.045 99.3475) (size 1.5) (drill 0.9) (layers F.Cu B.Cu) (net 20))
 (segment (start 137.43 98.97) (end 137.43 102.78) (width 0.8) (layer B.Cu) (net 20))
 (via (at 137.43 98.97) (size 1.5) (drill 0.9) (layers F.Cu B.Cu) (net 20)))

